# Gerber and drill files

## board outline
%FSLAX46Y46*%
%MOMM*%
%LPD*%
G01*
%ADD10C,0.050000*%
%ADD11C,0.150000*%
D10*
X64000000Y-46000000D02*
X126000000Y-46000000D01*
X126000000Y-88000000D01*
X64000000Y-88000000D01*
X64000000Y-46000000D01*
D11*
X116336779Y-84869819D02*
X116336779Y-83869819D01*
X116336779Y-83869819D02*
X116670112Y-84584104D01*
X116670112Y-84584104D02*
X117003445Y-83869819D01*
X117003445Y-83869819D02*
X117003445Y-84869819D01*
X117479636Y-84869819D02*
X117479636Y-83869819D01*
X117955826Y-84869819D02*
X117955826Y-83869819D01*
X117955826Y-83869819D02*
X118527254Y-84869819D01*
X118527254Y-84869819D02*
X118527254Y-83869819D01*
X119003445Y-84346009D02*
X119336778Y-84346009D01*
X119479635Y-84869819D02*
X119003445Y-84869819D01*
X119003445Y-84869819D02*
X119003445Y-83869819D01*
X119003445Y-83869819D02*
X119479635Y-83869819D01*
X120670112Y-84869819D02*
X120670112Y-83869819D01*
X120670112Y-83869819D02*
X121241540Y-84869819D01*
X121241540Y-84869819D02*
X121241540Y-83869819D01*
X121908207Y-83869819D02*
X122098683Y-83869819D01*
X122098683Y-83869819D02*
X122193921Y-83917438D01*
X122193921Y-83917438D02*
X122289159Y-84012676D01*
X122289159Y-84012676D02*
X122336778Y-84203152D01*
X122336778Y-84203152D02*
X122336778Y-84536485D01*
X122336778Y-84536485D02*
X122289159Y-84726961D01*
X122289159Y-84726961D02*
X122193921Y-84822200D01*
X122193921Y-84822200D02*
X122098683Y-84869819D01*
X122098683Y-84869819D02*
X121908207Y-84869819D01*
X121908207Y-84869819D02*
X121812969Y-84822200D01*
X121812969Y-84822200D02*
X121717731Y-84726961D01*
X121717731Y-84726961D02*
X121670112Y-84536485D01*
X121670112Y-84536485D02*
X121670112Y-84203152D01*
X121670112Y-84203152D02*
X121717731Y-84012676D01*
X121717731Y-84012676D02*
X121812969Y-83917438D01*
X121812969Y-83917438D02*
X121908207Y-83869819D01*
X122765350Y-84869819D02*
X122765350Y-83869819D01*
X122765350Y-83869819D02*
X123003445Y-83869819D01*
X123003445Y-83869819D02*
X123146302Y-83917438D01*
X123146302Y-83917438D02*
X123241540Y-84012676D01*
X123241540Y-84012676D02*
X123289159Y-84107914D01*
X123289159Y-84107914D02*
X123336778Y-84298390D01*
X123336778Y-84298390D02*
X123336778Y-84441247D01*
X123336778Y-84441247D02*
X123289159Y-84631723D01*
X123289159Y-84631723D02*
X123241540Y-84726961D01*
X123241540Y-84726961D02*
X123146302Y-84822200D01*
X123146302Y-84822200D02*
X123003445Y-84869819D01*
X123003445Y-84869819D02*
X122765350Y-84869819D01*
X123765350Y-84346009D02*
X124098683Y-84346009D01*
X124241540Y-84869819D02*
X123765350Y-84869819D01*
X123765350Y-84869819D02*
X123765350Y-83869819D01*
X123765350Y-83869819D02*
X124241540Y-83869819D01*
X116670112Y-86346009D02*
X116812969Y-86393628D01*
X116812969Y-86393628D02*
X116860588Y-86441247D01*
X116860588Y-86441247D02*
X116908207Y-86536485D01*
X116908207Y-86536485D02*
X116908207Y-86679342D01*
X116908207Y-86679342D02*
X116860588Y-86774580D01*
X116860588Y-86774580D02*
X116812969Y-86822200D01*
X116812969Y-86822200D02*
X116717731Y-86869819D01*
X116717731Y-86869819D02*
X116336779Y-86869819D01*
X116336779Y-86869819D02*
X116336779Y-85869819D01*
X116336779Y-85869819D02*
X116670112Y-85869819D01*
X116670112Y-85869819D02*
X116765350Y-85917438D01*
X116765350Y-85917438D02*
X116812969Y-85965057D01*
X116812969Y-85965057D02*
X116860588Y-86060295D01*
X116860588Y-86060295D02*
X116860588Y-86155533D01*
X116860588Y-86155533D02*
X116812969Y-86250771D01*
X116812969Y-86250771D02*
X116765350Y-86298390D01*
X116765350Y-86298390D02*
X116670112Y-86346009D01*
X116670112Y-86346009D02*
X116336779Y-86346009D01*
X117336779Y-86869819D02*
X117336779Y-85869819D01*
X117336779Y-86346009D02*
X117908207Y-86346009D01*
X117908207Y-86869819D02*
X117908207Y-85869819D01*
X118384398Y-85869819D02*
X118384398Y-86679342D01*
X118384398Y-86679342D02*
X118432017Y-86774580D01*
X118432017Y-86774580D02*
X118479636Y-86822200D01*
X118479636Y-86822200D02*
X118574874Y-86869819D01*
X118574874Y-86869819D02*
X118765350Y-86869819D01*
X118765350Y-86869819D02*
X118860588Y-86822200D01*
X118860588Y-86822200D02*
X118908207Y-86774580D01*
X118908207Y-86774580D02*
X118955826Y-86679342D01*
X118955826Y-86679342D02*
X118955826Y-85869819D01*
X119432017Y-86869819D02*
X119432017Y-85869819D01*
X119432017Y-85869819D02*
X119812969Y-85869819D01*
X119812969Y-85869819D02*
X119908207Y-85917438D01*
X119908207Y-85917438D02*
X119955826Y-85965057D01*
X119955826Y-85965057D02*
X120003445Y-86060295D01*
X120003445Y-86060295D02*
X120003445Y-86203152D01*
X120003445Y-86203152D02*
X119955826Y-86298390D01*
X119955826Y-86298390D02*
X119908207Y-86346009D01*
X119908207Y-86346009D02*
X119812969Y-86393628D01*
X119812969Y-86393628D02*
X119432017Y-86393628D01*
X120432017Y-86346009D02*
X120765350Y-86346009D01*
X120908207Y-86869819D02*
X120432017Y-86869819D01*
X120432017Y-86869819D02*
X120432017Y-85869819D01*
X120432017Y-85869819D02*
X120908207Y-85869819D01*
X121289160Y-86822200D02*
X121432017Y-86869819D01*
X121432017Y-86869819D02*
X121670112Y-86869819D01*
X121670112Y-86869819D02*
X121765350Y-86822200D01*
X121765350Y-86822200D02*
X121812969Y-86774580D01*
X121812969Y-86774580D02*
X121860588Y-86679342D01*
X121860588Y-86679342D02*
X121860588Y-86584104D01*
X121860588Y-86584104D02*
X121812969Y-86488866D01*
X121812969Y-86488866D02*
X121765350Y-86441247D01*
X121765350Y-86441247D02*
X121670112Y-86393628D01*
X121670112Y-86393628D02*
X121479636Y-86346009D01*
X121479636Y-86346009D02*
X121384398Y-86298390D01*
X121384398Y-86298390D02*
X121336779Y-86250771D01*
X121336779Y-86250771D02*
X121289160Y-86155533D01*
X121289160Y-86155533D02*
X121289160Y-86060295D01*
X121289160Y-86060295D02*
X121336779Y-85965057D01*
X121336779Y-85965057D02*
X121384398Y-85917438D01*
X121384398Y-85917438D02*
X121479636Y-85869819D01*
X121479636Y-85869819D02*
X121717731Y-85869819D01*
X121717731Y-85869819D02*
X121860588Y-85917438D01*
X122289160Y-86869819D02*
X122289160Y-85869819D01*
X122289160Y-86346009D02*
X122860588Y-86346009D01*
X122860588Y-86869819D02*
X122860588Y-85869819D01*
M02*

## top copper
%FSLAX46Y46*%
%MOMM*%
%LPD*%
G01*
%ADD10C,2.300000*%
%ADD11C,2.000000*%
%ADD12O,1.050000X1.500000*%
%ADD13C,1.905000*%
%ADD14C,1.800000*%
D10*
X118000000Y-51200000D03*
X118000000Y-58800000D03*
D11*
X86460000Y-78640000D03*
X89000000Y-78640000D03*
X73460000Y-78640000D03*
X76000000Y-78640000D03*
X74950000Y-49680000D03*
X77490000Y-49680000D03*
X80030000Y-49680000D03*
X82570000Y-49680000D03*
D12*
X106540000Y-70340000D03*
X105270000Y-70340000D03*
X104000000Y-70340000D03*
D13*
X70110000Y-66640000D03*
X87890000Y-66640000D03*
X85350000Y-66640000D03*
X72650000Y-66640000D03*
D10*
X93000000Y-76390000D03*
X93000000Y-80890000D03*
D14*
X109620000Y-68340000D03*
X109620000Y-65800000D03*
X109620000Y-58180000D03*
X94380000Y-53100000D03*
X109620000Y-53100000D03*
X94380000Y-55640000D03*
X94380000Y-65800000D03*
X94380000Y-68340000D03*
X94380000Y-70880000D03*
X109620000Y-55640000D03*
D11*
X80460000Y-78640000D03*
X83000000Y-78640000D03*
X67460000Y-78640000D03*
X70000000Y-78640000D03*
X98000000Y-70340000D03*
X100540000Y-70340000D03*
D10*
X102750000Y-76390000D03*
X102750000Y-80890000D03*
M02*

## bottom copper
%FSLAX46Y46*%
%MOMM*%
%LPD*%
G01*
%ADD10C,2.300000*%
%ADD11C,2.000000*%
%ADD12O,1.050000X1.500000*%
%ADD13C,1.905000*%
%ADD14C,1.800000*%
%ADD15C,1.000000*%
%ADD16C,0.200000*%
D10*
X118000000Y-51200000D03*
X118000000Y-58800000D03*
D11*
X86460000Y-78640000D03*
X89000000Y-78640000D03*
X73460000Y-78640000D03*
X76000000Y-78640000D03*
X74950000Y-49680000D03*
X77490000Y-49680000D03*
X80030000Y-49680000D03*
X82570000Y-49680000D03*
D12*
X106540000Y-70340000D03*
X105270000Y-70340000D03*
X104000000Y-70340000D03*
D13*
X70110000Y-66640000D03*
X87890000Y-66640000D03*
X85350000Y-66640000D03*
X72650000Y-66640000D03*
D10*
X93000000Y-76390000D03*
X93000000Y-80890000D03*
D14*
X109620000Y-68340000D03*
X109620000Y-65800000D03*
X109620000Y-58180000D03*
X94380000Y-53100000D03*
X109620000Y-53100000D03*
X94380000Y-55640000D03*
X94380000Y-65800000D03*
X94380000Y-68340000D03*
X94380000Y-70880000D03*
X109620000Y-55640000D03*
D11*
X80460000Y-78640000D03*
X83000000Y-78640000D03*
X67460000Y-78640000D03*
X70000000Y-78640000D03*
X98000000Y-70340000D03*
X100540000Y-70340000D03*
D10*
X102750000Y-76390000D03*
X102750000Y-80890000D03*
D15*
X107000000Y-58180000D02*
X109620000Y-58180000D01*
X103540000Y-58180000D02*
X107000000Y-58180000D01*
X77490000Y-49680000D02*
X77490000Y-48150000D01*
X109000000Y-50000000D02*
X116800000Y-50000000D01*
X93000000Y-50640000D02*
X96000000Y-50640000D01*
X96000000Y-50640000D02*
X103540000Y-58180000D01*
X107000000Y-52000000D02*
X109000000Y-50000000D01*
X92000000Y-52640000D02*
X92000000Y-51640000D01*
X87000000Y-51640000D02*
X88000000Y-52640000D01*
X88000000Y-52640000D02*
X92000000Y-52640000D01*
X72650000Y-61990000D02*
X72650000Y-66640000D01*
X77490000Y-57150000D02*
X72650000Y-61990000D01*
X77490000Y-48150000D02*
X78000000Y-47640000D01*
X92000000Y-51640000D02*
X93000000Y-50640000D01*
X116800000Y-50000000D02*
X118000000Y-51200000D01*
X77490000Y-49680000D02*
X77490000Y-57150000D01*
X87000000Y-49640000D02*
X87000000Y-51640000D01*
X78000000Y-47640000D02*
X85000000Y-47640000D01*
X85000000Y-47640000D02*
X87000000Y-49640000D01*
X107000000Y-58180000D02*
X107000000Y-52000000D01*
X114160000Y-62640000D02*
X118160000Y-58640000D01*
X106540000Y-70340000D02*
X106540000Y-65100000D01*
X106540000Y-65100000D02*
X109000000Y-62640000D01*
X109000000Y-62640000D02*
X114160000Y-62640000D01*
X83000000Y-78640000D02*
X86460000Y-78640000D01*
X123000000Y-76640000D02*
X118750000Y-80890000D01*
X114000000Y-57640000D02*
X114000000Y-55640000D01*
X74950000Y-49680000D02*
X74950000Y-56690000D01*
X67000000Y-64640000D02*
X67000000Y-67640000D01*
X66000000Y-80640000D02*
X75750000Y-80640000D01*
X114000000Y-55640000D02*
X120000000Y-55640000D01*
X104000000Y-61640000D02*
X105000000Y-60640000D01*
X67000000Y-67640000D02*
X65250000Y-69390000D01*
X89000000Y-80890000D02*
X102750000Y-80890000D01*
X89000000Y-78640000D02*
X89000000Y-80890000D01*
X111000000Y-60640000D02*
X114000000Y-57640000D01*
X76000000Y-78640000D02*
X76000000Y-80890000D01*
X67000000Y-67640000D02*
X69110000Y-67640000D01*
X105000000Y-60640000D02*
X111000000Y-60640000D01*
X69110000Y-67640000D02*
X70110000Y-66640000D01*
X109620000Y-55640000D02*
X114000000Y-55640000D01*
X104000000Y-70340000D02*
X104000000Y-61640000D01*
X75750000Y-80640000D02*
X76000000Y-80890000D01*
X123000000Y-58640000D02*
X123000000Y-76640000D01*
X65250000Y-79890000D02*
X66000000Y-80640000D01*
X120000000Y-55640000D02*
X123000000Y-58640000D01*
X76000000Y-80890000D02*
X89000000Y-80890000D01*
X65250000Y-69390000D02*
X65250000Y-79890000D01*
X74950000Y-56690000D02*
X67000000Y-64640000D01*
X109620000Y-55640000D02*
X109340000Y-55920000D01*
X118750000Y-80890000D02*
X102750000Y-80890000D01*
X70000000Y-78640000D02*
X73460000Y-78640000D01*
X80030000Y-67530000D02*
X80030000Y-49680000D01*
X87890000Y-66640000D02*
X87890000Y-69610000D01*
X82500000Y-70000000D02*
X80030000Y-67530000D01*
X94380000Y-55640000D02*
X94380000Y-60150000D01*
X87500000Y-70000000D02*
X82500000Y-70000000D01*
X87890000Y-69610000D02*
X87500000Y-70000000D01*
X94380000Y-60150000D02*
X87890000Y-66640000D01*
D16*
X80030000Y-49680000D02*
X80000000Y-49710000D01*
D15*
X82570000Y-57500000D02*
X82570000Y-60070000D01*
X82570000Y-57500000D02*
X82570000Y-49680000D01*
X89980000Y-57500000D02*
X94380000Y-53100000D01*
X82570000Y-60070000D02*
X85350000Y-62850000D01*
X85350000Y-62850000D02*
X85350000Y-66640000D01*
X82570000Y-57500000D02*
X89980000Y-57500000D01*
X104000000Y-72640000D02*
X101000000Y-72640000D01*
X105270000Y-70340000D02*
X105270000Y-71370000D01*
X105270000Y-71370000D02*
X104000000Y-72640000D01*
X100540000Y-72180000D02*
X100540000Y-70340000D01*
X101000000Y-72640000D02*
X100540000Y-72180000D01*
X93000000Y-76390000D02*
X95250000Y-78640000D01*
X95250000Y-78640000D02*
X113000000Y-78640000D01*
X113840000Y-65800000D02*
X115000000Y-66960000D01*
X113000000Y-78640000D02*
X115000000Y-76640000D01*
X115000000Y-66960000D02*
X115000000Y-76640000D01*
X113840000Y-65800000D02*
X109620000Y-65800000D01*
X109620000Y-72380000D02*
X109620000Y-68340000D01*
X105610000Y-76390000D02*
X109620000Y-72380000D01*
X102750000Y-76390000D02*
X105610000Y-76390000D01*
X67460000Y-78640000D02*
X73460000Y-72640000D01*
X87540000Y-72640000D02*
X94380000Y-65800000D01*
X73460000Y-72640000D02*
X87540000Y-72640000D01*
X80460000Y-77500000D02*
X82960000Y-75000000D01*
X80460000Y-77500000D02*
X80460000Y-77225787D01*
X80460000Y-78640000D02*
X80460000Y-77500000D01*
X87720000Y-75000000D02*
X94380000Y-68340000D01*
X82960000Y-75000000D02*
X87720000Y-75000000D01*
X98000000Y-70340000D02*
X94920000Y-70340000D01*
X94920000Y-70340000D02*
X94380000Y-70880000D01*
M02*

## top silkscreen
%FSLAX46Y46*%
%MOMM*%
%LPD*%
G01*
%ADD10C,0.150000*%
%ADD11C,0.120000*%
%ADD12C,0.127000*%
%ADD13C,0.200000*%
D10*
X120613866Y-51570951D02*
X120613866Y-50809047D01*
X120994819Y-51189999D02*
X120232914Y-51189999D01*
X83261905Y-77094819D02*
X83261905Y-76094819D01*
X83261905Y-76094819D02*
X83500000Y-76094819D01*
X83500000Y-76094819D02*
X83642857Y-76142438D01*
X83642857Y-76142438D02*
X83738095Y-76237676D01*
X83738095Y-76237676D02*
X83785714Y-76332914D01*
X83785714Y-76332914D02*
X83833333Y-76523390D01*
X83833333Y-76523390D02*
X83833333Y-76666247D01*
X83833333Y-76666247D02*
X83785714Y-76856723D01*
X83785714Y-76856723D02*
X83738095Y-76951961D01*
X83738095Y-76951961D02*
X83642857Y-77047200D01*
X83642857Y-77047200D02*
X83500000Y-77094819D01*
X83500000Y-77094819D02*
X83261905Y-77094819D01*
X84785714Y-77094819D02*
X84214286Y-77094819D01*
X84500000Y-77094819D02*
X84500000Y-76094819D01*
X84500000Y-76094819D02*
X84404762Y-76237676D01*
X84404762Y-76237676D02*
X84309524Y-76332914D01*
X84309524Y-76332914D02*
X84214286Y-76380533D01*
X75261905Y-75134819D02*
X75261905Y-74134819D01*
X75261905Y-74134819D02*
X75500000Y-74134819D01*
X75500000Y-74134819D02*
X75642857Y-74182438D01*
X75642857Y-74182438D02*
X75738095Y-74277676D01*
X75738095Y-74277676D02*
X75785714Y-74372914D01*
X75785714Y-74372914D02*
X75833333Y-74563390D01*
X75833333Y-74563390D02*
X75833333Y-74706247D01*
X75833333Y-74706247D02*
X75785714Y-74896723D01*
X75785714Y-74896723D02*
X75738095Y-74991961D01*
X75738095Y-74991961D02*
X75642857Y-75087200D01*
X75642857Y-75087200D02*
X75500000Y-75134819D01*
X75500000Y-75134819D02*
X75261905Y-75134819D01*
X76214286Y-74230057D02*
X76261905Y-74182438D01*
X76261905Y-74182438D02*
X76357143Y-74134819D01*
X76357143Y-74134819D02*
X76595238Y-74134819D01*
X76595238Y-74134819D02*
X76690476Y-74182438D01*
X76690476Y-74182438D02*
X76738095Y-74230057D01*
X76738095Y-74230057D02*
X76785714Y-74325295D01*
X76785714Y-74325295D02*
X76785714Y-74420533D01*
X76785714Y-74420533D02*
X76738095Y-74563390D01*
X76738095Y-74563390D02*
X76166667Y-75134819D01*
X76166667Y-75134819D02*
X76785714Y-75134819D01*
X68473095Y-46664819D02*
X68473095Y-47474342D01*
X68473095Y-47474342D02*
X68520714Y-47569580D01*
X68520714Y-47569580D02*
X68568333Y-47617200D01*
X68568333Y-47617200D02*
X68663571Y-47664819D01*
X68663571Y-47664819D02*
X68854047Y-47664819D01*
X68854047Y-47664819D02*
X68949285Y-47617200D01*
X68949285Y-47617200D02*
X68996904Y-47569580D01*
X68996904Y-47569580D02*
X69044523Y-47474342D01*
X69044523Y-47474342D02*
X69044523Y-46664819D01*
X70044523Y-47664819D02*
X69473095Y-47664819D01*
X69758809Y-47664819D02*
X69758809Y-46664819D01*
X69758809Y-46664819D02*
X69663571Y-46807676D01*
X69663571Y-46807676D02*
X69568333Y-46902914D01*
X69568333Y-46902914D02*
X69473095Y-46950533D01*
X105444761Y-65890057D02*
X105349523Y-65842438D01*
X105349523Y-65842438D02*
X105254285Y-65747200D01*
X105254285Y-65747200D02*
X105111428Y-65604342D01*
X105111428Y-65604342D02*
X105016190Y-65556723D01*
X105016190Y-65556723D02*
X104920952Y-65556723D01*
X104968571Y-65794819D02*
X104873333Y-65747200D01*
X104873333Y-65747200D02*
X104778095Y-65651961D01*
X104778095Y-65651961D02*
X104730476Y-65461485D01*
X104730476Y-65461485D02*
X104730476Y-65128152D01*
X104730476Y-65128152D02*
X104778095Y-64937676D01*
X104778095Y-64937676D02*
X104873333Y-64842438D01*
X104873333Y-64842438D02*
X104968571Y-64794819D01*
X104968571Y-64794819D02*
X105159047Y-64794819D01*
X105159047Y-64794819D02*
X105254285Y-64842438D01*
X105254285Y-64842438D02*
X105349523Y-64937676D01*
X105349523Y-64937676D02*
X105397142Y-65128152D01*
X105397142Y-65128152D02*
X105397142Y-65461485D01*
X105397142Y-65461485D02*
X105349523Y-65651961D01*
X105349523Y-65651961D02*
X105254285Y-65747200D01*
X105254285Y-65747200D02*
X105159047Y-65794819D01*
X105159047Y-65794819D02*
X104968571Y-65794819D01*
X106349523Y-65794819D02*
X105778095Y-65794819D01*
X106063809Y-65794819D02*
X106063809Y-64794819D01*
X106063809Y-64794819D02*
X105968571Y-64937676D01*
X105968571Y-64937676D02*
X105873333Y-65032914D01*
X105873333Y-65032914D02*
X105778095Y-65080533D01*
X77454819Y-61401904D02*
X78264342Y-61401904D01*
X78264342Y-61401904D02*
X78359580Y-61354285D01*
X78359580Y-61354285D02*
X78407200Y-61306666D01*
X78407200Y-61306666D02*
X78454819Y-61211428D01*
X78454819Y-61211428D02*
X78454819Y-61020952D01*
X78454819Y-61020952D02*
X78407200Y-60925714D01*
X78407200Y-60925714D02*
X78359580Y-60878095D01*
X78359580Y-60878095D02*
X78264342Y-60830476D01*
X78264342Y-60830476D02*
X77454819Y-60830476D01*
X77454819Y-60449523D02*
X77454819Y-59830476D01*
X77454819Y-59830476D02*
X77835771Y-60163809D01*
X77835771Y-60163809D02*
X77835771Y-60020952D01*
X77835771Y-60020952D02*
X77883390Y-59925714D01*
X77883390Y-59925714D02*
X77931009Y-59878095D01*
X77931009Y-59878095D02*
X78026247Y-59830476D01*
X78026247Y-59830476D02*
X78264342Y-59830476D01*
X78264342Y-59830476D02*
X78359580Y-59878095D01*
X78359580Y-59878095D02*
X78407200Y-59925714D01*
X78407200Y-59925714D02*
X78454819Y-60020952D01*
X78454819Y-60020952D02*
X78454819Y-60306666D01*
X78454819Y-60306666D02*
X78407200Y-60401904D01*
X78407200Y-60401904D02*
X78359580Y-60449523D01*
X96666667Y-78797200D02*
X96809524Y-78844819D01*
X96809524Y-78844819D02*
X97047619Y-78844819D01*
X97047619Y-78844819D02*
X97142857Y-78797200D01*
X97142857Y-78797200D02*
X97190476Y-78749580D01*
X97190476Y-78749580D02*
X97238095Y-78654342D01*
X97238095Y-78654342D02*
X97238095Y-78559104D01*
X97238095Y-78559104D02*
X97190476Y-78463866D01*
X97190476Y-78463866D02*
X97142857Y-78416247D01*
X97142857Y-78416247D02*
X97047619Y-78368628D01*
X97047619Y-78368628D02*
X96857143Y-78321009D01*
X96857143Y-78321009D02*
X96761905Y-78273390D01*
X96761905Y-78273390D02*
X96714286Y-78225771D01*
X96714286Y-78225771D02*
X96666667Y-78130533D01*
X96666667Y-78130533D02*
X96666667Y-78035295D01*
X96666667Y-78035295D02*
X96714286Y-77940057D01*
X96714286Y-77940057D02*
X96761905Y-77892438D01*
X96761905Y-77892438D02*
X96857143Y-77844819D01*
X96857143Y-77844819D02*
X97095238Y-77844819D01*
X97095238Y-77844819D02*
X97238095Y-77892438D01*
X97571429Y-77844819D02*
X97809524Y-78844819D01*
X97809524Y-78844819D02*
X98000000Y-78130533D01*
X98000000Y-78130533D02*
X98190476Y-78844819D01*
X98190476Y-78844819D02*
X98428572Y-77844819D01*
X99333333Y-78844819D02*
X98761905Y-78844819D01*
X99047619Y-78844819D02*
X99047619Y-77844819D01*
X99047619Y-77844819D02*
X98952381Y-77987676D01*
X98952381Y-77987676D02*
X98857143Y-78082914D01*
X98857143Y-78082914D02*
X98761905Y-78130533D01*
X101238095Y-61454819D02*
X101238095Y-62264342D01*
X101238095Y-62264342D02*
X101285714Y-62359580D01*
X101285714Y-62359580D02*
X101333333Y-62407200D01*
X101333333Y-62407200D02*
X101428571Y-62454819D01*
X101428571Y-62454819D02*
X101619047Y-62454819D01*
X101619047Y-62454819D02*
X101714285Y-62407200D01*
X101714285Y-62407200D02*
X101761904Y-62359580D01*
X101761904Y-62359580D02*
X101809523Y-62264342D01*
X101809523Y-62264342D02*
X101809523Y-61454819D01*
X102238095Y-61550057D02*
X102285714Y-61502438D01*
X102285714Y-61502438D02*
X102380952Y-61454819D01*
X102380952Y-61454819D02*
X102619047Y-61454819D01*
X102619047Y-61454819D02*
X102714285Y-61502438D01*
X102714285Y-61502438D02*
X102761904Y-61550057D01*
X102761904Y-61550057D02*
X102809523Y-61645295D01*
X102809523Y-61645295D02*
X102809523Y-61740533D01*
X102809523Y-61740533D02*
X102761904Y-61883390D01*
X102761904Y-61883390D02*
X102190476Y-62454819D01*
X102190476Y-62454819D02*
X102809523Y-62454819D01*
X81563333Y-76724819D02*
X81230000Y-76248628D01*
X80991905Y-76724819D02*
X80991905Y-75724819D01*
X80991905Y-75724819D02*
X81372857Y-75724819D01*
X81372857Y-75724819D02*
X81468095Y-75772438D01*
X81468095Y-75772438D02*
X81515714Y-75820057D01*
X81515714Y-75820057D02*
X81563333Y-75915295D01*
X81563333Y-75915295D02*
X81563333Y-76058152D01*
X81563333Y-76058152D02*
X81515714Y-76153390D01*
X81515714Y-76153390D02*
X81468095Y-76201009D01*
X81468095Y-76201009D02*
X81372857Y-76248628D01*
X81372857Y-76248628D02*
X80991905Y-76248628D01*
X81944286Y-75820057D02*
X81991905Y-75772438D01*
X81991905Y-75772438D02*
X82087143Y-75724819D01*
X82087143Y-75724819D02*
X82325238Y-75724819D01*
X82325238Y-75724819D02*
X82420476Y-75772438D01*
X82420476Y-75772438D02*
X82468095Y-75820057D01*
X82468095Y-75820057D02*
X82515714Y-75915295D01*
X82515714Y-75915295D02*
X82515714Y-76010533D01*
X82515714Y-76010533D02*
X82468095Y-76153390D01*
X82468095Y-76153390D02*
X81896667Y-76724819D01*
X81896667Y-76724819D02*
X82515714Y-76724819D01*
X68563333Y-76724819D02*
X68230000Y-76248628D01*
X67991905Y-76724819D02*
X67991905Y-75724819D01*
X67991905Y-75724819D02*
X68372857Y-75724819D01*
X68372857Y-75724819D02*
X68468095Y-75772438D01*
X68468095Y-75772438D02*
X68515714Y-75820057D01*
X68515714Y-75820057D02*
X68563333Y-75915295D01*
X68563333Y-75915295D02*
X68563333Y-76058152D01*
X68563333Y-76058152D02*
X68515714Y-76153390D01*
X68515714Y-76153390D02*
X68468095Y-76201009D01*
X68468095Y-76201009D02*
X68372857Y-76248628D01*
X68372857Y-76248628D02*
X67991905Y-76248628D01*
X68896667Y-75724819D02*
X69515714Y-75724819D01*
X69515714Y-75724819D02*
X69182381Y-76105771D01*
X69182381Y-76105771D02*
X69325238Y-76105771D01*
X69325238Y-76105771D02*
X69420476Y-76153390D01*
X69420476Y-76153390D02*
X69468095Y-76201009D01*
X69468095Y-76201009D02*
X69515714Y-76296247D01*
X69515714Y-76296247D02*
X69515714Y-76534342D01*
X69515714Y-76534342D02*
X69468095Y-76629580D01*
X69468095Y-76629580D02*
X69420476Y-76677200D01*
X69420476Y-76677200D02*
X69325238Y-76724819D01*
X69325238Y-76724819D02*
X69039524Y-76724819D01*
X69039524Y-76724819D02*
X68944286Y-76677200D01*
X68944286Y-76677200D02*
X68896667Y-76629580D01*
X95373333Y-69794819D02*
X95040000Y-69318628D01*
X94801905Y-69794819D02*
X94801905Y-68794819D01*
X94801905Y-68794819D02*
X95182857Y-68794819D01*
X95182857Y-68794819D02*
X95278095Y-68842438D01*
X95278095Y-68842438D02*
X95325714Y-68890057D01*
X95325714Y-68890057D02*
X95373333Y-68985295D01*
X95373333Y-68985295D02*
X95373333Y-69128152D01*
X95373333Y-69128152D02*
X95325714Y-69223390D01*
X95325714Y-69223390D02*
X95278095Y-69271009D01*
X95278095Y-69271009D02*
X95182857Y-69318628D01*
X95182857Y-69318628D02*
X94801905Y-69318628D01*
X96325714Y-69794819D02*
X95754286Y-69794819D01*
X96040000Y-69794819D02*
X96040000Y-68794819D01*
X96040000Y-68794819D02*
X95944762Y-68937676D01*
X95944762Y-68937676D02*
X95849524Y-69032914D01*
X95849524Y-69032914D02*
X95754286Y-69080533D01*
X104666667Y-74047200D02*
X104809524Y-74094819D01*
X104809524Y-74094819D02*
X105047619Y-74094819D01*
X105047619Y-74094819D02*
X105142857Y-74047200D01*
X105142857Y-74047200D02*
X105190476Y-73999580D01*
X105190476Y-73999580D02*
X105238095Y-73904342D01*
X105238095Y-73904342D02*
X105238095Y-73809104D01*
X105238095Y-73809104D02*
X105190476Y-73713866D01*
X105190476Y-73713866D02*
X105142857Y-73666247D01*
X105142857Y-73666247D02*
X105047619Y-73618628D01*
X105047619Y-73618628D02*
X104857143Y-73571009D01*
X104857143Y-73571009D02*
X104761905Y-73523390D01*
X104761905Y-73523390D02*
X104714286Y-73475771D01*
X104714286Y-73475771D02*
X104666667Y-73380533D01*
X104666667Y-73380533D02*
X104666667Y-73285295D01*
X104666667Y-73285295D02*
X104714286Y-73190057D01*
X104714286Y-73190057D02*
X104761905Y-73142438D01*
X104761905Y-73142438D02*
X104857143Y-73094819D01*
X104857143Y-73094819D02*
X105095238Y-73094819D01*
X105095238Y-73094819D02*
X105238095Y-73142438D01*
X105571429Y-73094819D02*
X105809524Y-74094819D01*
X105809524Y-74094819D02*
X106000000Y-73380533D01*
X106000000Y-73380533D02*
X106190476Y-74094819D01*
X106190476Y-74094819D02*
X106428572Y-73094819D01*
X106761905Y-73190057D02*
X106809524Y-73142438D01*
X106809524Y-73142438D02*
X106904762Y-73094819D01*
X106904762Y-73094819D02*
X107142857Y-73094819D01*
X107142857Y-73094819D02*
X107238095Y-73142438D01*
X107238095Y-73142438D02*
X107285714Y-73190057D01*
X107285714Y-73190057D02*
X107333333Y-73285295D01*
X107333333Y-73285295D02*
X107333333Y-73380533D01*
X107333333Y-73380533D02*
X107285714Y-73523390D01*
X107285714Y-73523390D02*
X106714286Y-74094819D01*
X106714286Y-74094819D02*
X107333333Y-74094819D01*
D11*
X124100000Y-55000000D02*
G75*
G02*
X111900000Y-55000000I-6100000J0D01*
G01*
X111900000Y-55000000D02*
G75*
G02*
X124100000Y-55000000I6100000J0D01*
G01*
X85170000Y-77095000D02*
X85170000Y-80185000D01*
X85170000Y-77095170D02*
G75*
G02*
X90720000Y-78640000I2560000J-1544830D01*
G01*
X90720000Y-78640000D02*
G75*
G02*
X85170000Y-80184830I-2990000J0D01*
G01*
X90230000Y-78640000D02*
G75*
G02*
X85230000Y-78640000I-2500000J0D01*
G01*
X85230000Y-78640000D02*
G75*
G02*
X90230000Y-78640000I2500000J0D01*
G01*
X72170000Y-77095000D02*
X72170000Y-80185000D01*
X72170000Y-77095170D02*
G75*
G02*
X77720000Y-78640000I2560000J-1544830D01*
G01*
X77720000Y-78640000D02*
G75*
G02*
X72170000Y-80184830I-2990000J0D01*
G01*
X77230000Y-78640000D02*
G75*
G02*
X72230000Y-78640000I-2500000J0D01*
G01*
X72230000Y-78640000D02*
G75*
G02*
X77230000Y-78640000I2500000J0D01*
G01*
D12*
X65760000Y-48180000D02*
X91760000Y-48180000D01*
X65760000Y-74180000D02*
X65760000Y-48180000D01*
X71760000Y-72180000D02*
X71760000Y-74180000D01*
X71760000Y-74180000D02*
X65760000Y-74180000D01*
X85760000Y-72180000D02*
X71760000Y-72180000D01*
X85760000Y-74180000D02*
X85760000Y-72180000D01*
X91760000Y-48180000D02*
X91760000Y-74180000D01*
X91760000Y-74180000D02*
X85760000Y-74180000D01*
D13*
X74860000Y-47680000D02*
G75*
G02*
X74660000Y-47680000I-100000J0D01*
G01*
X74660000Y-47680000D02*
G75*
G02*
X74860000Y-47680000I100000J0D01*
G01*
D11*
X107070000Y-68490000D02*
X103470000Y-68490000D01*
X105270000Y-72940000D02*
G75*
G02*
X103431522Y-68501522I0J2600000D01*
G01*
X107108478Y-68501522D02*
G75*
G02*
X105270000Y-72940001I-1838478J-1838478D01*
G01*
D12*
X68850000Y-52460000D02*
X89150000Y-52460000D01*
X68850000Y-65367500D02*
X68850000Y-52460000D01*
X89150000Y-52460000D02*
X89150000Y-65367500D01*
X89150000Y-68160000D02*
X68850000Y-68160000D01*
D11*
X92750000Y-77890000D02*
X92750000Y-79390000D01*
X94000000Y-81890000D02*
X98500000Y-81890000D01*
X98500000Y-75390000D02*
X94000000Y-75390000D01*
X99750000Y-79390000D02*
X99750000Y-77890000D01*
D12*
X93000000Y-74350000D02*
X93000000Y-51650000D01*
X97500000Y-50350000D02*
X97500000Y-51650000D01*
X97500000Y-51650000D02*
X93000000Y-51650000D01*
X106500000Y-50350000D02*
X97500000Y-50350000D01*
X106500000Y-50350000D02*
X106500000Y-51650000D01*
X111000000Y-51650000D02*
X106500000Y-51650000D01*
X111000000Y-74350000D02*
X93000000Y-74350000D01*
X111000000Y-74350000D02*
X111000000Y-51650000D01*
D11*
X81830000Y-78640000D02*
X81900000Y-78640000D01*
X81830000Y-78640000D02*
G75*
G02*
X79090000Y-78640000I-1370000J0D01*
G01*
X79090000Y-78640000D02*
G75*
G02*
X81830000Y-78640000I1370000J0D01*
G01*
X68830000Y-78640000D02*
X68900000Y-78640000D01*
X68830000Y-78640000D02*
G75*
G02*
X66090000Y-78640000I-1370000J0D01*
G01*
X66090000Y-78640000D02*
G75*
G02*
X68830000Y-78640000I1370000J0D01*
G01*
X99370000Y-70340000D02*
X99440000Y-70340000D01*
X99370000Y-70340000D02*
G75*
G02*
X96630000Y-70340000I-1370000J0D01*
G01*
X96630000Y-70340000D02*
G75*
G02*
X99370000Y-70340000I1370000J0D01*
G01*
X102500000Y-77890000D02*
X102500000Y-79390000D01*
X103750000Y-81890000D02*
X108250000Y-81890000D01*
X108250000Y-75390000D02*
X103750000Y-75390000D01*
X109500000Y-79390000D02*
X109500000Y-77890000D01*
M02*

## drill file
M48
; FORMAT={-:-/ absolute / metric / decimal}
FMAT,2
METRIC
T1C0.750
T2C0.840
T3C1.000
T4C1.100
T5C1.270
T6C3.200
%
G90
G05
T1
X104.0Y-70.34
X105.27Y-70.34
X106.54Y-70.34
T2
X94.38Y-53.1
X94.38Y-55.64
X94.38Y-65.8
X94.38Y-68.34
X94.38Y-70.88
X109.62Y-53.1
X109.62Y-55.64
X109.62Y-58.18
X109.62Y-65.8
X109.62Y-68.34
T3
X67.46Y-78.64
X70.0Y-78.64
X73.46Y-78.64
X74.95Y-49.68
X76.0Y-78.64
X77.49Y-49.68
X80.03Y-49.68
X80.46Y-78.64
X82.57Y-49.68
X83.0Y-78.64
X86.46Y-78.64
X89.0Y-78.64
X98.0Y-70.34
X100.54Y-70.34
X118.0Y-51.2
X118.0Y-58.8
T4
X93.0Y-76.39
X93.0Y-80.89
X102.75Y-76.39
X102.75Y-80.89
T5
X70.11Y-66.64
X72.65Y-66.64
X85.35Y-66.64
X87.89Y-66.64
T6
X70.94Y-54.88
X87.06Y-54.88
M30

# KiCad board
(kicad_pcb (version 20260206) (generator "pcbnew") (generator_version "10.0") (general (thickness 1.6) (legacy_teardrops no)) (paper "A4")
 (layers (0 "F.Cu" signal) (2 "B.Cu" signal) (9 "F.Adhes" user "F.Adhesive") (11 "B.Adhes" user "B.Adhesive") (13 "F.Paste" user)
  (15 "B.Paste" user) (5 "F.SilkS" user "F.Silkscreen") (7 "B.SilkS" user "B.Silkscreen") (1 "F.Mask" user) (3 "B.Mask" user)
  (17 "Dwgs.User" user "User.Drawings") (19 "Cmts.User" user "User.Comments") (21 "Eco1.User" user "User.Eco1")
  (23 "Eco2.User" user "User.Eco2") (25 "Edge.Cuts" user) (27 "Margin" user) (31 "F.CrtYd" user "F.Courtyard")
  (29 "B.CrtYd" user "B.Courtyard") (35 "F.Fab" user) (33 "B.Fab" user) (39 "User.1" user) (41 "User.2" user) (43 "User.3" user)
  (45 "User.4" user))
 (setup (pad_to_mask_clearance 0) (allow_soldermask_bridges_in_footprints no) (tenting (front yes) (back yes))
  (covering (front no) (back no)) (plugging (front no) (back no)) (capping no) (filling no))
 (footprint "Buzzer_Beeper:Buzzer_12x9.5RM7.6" (layer "F.Cu") (at 118 51.2 -90)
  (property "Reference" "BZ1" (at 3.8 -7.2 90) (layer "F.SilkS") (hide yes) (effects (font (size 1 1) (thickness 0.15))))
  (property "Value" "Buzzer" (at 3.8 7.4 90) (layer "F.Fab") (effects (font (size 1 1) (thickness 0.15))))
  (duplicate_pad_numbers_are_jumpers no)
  (fp_circle (center 3.8 0) (end 9.9 0) (stroke (width 0.12) (type solid)) (fill no) (layer "F.SilkS"))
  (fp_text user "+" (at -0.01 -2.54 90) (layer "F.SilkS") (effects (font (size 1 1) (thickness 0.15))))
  (pad "1" thru_hole circle (at 0 0 270) (size 2.3 2.3) (drill 1) (layers "*.Cu" "*.Mask") (remove_unused_layers no) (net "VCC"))
  (pad "2" thru_hole circle (at 7.6 0 270) (size 2.3 2.3) (drill 1) (layers "*.Cu" "*.Mask") (remove_unused_layers no) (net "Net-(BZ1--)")))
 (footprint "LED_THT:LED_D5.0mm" (layer "F.Cu") (at 86.46 78.64)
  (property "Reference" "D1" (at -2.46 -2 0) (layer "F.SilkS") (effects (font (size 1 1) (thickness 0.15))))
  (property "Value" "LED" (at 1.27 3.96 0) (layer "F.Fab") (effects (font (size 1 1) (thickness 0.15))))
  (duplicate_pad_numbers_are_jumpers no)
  (fp_line (start -1.29 -1.545) (end -1.29 1.545) (stroke (width 0.12) (type solid)) (layer "F.SilkS"))
  (fp_arc (start -1.29 -1.54483) (mid 2.071779 -2.880495) (end 4.26 0) (stroke (width 0.12) (type solid)) (layer "F.SilkS"))
  (fp_arc (start 4.26 0) (mid 2.071779 2.880495) (end -1.29 1.54483) (stroke (width 0.12) (type solid)) (layer "F.SilkS"))
  (fp_circle (center 1.27 0) (end 3.77 0) (stroke (width 0.12) (type solid)) (fill no) (layer "F.SilkS"))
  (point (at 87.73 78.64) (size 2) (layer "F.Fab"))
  (pad "1" thru_hole circle (at 0 0) (size 2 2) (drill 1) (layers "*.Cu" "*.Mask") (remove_unused_layers no) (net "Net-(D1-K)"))
  (pad "2" thru_hole circle (at 2.54 0) (size 2 2) (drill 1) (layers "*.Cu" "*.Mask") (remove_unused_layers no) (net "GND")))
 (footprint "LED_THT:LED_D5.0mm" (layer "F.Cu") (at 73.46 78.64)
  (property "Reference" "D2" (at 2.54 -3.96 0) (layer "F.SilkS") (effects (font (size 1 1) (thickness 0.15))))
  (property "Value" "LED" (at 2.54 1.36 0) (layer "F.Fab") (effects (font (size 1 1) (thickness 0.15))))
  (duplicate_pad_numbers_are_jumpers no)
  (fp_line (start -1.29 -1.545) (end -1.29 1.545) (stroke (width 0.12) (type solid)) (layer "F.SilkS"))
  (fp_arc (start -1.29 -1.54483) (mid 2.071779 -2.880495) (end 4.26 0) (stroke (width 0.12) (type solid)) (layer "F.SilkS"))
  (fp_arc (start 4.26 0) (mid 2.071779 2.880495) (end -1.29 1.54483) (stroke (width 0.12) (type solid)) (layer "F.SilkS"))
  (fp_circle (center 1.27 0) (end 3.77 0) (stroke (width 0.12) (type solid)) (fill no) (layer "F.SilkS"))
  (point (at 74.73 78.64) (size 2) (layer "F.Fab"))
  (pad "1" thru_hole circle (at 0 0) (size 2 2) (drill 1) (layers "*.Cu" "*.Mask") (remove_unused_layers no) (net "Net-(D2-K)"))
  (pad "2" thru_hole circle (at 2.54 0) (size 2 2) (drill 1) (layers "*.Cu" "*.Mask") (remove_unused_layers no) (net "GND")))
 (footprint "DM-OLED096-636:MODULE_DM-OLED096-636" (layer "F.Cu") (at 78.76 61.18)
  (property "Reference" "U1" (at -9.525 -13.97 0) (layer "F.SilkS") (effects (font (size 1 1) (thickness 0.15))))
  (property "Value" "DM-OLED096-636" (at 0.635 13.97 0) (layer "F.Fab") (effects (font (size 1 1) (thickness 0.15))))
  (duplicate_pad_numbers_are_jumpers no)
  (fp_line (start -13 -13) (end 13 -13) (stroke (width 0.127) (type solid)) (layer "F.SilkS"))
  (fp_line (start -13 13) (end -13 -13) (stroke (width 0.127) (type solid)) (layer "F.SilkS"))
  (fp_line (start -7 11) (end -7 13) (stroke (width 0.127) (type solid)) (layer "F.SilkS"))
  (fp_line (start -7 13) (end -13 13) (stroke (width 0.127) (type solid)) (layer "F.SilkS"))
  (fp_line (start 7 11) (end -7 11) (stroke (width 0.127) (type solid)) (layer "F.SilkS"))
  (fp_line (start 7 13) (end 7 11) (stroke (width 0.127) (type solid)) (layer "F.SilkS"))
  (fp_line (start 13 -13) (end 13 13) (stroke (width 0.127) (type solid)) (layer "F.SilkS"))
  (fp_line (start 13 13) (end 7 13) (stroke (width 0.127) (type solid)) (layer "F.SilkS"))
  (fp_circle (center -4 -13.5) (end -3.9 -13.5) (stroke (width 0.2) (type solid)) (fill no) (layer "F.SilkS"))
  (pad "1" thru_hole circle (at -3.81 -11.5) (size 2 2) (drill 1) (layers "*.Cu" "*.Mask") (remove_unused_layers no) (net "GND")
   (solder_mask_margin 0.102))
  (pad "2" thru_hole circle (at -1.27 -11.5) (size 2 2) (drill 1) (layers "*.Cu" "*.Mask") (remove_unused_layers no) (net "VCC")
   (solder_mask_margin 0.102))
  (pad "3" thru_hole circle (at 1.27 -11.5) (size 2 2) (drill 1) (layers "*.Cu" "*.Mask") (remove_unused_layers no) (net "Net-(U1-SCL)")
   (solder_mask_margin 0.102))
  (pad "4" thru_hole circle (at 3.81 -11.5) (size 2 2) (drill 1) (layers "*.Cu" "*.Mask") (remove_unused_layers no) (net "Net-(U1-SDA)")
   (solder_mask_margin 0.102)))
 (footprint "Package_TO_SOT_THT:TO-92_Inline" (layer "F.Cu") (at 106.54 70.34 180)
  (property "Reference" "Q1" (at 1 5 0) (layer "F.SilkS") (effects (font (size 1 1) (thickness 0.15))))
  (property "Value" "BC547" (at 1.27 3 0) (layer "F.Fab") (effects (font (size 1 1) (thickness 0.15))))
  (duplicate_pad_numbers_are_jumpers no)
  (fp_line (start -0.53 1.85) (end 3.07 1.85) (stroke (width 0.12) (type solid)) (layer "F.SilkS"))
  (fp_arc (start 1.27 -2.6) (mid 3.672087 -0.994977) (end 3.108478 1.838478) (stroke (width 0.12) (type solid)) (layer "F.SilkS"))
  (fp_arc (start -0.568478 1.838478) (mid -1.132087 -0.994977) (end 1.27 -2.6) (stroke (width 0.12) (type solid)) (layer "F.SilkS"))
  (pad "1" thru_hole oval (at 0 0 180) (size 1.05 1.5) (drill 0.75) (layers "*.Cu" "*.Mask") (remove_unused_layers no) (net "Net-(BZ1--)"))
  (pad "2" thru_hole oval (at 1.27 0 180) (size 1.05 1.5) (drill 0.75) (layers "*.Cu" "*.Mask") (remove_unused_layers no) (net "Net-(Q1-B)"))
  (pad "3" thru_hole oval (at 2.54 0 180) (size 1.05 1.5) (drill 0.75) (layers "*.Cu" "*.Mask") (remove_unused_layers no) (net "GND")))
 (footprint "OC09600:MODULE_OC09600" (layer "F.Cu") (at 79 60.31 90)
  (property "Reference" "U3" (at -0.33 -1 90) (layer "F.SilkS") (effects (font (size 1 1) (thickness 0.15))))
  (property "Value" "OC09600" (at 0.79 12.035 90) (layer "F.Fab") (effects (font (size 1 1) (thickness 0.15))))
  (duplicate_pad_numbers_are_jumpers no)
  (fp_line (start 7.85 -10.15) (end 7.85 10.15) (stroke (width 0.127) (type solid)) (layer "F.SilkS"))
  (fp_line (start -5.0575 -10.15) (end 7.85 -10.15) (stroke (width 0.127) (type solid)) (layer "F.SilkS"))
  (fp_line (start 7.85 10.15) (end -5.0575 10.15) (stroke (width 0.127) (type solid)) (layer "F.SilkS"))
  (fp_line (start -7.85 10.15) (end -7.85 -10.15) (stroke (width 0.127) (type solid)) (layer "F.SilkS"))
  (pad "" np_thru_hole circle (at 5.43 -8.06 90) (size 3.2 3.2) (drill 3.2) (layers "*.Cu" "*.Mask"))
  (pad "" np_thru_hole circle (at 5.43 8.06 90) (size 3.2 3.2) (drill 3.2) (layers "*.Cu" "*.Mask"))
  (pad "GND" thru_hole circle (at -6.33 -8.89 90) (size 1.905 1.905) (drill 1.27) (layers "*.Cu" "*.Mask") (remove_unused_layers no)
   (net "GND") (solder_mask_margin 0.102))
  (pad "SCL" thru_hole circle (at -6.33 8.89 90) (size 1.905 1.905) (drill 1.27) (layers "*.Cu" "*.Mask") (remove_unused_layers no)
   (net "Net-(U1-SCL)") (solder_mask_margin 0.102))
  (pad "SDA" thru_hole circle (at -6.33 6.35 90) (size 1.905 1.905) (drill 1.27) (layers "*.Cu" "*.Mask") (remove_unused_layers no)
   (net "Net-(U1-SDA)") (solder_mask_margin 0.102))
  (pad "VCC" thru_hole circle (at -6.33 -6.35 90) (size 1.905 1.905) (drill 1.27) (layers "*.Cu" "*.Mask") (remove_unused_layers no)
   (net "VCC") (solder_mask_margin 0.102)))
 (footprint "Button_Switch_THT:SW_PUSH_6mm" (layer "F.Cu") (at 93 76.39)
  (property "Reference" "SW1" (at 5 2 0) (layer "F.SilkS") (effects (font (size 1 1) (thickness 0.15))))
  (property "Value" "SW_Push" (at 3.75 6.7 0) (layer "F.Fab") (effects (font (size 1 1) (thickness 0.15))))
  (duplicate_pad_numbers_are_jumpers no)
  (fp_line (start -0.25 1.5) (end -0.25 3) (stroke (width 0.12) (type solid)) (layer "F.SilkS"))
  (fp_line (start 1 5.5) (end 5.5 5.5) (stroke (width 0.12) (type solid)) (layer "F.SilkS"))
  (fp_line (start 5.5 -1) (end 1 -1) (stroke (width 0.12) (type solid)) (layer "F.SilkS"))
  (fp_line (start 6.75 3) (end 6.75 1.5) (stroke (width 0.12) (type solid)) (layer "F.SilkS"))
  (pad "1" thru_hole circle (at 0 0 90) (size 2.3 2.3) (drill 1.1) (layers "*.Cu" "*.Mask") (remove_unused_layers no) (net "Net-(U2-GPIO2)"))
  (pad "2" thru_hole circle (at 0 4.5 90) (size 2.3 2.3) (drill 1.1) (layers "*.Cu" "*.Mask") (remove_unused_layers no) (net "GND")))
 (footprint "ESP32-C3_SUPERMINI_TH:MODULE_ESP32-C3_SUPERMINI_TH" (layer "F.Cu") (at 102 63)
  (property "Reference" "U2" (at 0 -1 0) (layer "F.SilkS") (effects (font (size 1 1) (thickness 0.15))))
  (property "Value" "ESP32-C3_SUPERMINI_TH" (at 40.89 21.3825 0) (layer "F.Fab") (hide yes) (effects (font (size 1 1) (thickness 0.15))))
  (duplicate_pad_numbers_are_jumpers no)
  (fp_line (start -9 11.35) (end -9 -11.35) (stroke (width 0.127) (type solid)) (layer "F.SilkS"))
  (fp_line (start -4.5 -12.65) (end -4.5 -11.35) (stroke (width 0.127) (type solid)) (layer "F.SilkS"))
  (fp_line (start -4.5 -11.35) (end -9 -11.35) (stroke (width 0.127) (type solid)) (layer "F.SilkS"))
  (fp_line (start 4.5 -12.65) (end -4.5 -12.65) (stroke (width 0.127) (type solid)) (layer "F.SilkS"))
  (fp_line (start 4.5 -12.65) (end 4.5 -11.35) (stroke (width 0.127) (type solid)) (layer "F.SilkS"))
  (fp_line (start 9 -11.35) (end 4.5 -11.35) (stroke (width 0.127) (type solid)) (layer "F.SilkS"))
  (fp_line (start 9 11.35) (end -9 11.35) (stroke (width 0.127) (type solid)) (layer "F.SilkS"))
  (fp_line (start 9 11.35) (end 9 -11.35) (stroke (width 0.127) (type solid)) (layer "F.SilkS"))
  (pad "1" thru_hole circle (at 7.62 5.34) (size 1.8 1.8) (drill 0.84) (layers "*.Cu" "*.Mask") (remove_unused_layers no)
   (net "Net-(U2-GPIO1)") (solder_mask_margin 0.102))
  (pad "2" thru_hole circle (at 7.62 2.8) (size 1.8 1.8) (drill 0.84) (layers "*.Cu" "*.Mask") (remove_unused_layers no)
   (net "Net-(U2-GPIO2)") (solder_mask_margin 0.102))
  (pad "3.3" thru_hole circle (at 7.62 -4.82) (size 1.8 1.8) (drill 0.84) (layers "*.Cu" "*.Mask") (remove_unused_layers no) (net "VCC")
   (solder_mask_margin 0.102))
  (pad "5" thru_hole circle (at -7.62 -9.9) (size 1.8 1.8) (drill 0.84) (layers "*.Cu" "*.Mask") (remove_unused_layers no)
   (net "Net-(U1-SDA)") (solder_mask_margin 0.102))
  (pad "5V" thru_hole circle (at 7.62 -9.9) (size 1.8 1.8) (drill 0.84) (layers "*.Cu" "*.Mask") (remove_unused_layers no)
   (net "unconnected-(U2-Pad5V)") (solder_mask_margin 0.102))
  (pad "6" thru_hole circle (at -7.62 -7.36) (size 1.8 1.8) (drill 0.84) (layers "*.Cu" "*.Mask") (remove_unused_layers no)
   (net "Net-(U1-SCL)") (solder_mask_margin 0.102))
  (pad "10" thru_hole circle (at -7.62 2.8) (size 1.8 1.8) (drill 0.84) (layers "*.Cu" "*.Mask") (remove_unused_layers no)
   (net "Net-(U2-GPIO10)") (solder_mask_margin 0.102))
  (pad "20" thru_hole circle (at -7.62 5.34) (size 1.8 1.8) (drill 0.84) (layers "*.Cu" "*.Mask") (remove_unused_layers no)
   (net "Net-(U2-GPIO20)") (solder_mask_margin 0.102))
  (pad "21" thru_hole circle (at -7.62 7.88) (size 1.8 1.8) (drill 0.84) (layers "*.Cu" "*.Mask") (remove_unused_layers no)
   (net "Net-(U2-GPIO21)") (solder_mask_margin 0.102))
  (pad "G" thru_hole circle (at 7.62 -7.36) (size 1.8 1.8) (drill 0.84) (layers "*.Cu" "*.Mask") (remove_unused_layers no) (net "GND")
   (solder_mask_margin 0.102)))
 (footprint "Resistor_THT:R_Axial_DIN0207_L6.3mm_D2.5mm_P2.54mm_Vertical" (layer "F.Cu") (at 80.46 78.64)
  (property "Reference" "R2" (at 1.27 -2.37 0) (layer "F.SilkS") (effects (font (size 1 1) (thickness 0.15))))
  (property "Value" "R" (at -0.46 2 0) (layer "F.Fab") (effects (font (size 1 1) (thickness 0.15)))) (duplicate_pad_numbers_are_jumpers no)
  (fp_line (start 1.37 0) (end 1.44 0) (stroke (width 0.12) (type solid)) (layer "F.SilkS"))
  (fp_circle (center 0 0) (end 1.37 0) (stroke (width 0.12) (type solid)) (fill no) (layer "F.SilkS"))
  (pad "1" thru_hole circle (at 0 0) (size 2 2) (drill 1) (layers "*.Cu" "*.Mask") (remove_unused_layers no) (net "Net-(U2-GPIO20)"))
  (pad "2" thru_hole circle (at 2.54 0) (size 2 2) (drill 1) (layers "*.Cu" "*.Mask") (remove_unused_layers no) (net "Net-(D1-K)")))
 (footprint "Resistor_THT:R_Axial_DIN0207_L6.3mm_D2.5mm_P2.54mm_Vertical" (layer "F.Cu") (at 67.46 78.64)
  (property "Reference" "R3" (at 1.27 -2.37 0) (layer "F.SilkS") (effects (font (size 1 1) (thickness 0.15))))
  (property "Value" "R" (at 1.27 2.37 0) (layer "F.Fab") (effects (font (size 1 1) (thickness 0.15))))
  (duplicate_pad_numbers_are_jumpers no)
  (fp_line (start 1.37 0) (end 1.44 0) (stroke (width 0.12) (type solid)) (layer "F.SilkS"))
  (fp_circle (center 0 0) (end 1.37 0) (stroke (width 0.12) (type solid)) (fill no) (layer "F.SilkS"))
  (pad "1" thru_hole circle (at 0 0) (size 2 2) (drill 1) (layers "*.Cu" "*.Mask") (remove_unused_layers no) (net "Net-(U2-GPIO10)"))
  (pad "2" thru_hole circle (at 2.54 0) (size 2 2) (drill 1) (layers "*.Cu" "*.Mask") (remove_unused_layers no) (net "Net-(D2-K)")))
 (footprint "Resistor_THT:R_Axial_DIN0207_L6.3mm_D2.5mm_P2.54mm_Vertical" (layer "F.Cu") (at 98 70.34)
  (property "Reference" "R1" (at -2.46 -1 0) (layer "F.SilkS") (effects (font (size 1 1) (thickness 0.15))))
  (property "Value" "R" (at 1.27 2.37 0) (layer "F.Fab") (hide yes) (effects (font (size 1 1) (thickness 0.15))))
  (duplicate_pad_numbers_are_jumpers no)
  (fp_line (start 1.37 0) (end 1.44 0) (stroke (width 0.12) (type solid)) (layer "F.SilkS"))
  (fp_circle (center 0 0) (end 1.37 0) (stroke (width 0.12) (type solid)) (fill no) (layer "F.SilkS"))
  (pad "1" thru_hole circle (at 0 0) (size 2 2) (drill 1) (layers "*.Cu" "*.Mask") (remove_unused_layers no) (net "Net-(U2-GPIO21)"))
  (pad "2" thru_hole circle (at 2.54 0) (size 2 2) (drill 1) (layers "*.Cu" "*.Mask") (remove_unused_layers no) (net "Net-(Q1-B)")))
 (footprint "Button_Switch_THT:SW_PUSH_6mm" (layer "F.Cu") (at 102.75 76.39)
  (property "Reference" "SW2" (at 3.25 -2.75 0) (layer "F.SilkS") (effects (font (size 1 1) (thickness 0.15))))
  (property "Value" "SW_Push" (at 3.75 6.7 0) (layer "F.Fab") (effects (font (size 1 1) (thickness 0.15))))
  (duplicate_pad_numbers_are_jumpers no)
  (fp_line (start -0.25 1.5) (end -0.25 3) (stroke (width 0.12) (type solid)) (layer "F.SilkS"))
  (fp_line (start 1 5.5) (end 5.5 5.5) (stroke (width 0.12) (type solid)) (layer "F.SilkS"))
  (fp_line (start 5.5 -1) (end 1 -1) (stroke (width 0.12) (type solid)) (layer "F.SilkS"))
  (fp_line (start 6.75 3) (end 6.75 1.5) (stroke (width 0.12) (type solid)) (layer "F.SilkS"))
  (pad "1" thru_hole circle (at 0 0 90) (size 2.3 2.3) (drill 1.1) (layers "*.Cu" "*.Mask") (remove_unused_layers no) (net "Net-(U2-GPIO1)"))
  (pad "2" thru_hole circle (at 0 4.5 90) (size 2.3 2.3) (drill 1.1) (layers "*.Cu" "*.Mask") (remove_unused_layers no) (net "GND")))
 (gr_rect (start 64 46) (end 126 88) (stroke (width 0.05) (type default)) (fill no) (layer "Edge.Cuts"))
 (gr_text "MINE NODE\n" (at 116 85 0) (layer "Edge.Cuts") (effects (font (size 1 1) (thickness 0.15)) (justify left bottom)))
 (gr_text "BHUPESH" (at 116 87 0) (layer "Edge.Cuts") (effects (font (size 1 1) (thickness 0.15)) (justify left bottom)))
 (segment (start 107 58.18) (end 109.62 58.18) (width 1) (layer "B.Cu") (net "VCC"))
 (segment (start 103.54 58.18) (end 107 58.18) (width 1) (layer "B.Cu") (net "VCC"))
 (segment (start 77.49 49.68) (end 77.49 48.15) (width 1) (layer "B.Cu") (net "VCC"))
 (segment (start 109 50) (end 116.8 50) (width 1) (layer "B.Cu") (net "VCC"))
 (segment (start 93 50.64) (end 96 50.64) (width 1) (layer "B.Cu") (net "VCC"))
 (segment (start 96 50.64) (end 103.54 58.18) (width 1) (layer "B.Cu") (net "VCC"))
 (segment (start 107 52) (end 109 50) (width 1) (layer "B.Cu") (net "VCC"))
 (segment (start 92 52.64) (end 92 51.64) (width 1) (layer "B.Cu") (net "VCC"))
 (segment (start 87 51.64) (end 88 52.64) (width 1) (layer "B.Cu") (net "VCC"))
 (segment (start 88 52.64) (end 92 52.64) (width 1) (layer "B.Cu") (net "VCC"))
 (segment (start 72.65 61.99) (end 72.65 66.64) (width 1) (layer "B.Cu") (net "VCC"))
 (segment (start 77.49 57.15) (end 72.65 61.99) (width 1) (layer "B.Cu") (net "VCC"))
 (segment (start 77.49 48.15) (end 78 47.64) (width 1) (layer "B.Cu") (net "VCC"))
 (segment (start 92 51.64) (end 93 50.64) (width 1) (layer "B.Cu") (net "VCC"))
 (segment (start 116.8 50) (end 118 51.2) (width 1) (layer "B.Cu") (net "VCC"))
 (segment (start 77.49 49.68) (end 77.49 57.15) (width 1) (layer "B.Cu") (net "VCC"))
 (segment (start 87 49.64) (end 87 51.64) (width 1) (layer "B.Cu") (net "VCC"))
 (segment (start 78 47.64) (end 85 47.64) (width 1) (layer "B.Cu") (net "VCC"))
 (segment (start 85 47.64) (end 87 49.64) (width 1) (layer "B.Cu") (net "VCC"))
 (segment (start 107 58.18) (end 107 52) (width 1) (layer "B.Cu") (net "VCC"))
 (segment (start 114.16 62.64) (end 118.16 58.64) (width 1) (layer "B.Cu") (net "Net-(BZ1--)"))
 (segment (start 106.54 70.34) (end 106.54 65.1) (width 1) (layer "B.Cu") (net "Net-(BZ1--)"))
 (segment (start 106.54 65.1) (end 109 62.64) (width 1) (layer "B.Cu") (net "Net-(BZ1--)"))
 (segment (start 109 62.64) (end 114.16 62.64) (width 1) (layer "B.Cu") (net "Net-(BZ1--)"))
 (segment (start 83 78.64) (end 86.46 78.64) (width 1) (layer "B.Cu") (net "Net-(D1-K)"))
 (segment (start 123 76.64) (end 118.75 80.89) (width 1) (layer "B.Cu") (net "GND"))
 (segment (start 114 57.64) (end 114 55.64) (width 1) (layer "B.Cu") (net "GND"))
 (segment (start 74.95 49.68) (end 74.95 56.69) (width 1) (layer "B.Cu") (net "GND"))
 (segment (start 67 64.64) (end 67 67.64) (width 1) (layer "B.Cu") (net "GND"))
 (segment (start 66 80.64) (end 75.75 80.64) (width 1) (layer "B.Cu") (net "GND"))
 (segment (start 114 55.64) (end 120 55.64) (width 1) (layer "B.Cu") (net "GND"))
 (segment (start 104 61.64) (end 105 60.64) (width 1) (layer "B.Cu") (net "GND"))
 (segment (start 67 67.64) (end 65.25 69.39) (width 1) (layer "B.Cu") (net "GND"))
 (segment (start 89 80.89) (end 102.75 80.89) (width 1) (layer "B.Cu") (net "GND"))
 (segment (start 89 78.64) (end 89 80.89) (width 1) (layer "B.Cu") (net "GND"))
 (segment (start 111 60.64) (end 114 57.64) (width 1) (layer "B.Cu") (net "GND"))
 (segment (start 76 78.64) (end 76 80.89) (width 1) (layer "B.Cu") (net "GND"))
 (segment (start 67 67.64) (end 69.11 67.64) (width 1) (layer "B.Cu") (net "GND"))
 (segment (start 105 60.64) (end 111 60.64) (width 1) (layer "B.Cu") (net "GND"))
 (segment (start 69.11 67.64) (end 70.11 66.64) (width 1) (layer "B.Cu") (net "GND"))
 (segment (start 109.62 55.64) (end 114 55.64) (width 1) (layer "B.Cu") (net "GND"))
 (segment (start 104 70.34) (end 104 61.64) (width 1) (layer "B.Cu") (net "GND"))
 (segment (start 75.75 80.64) (end 76 80.89) (width 1) (layer "B.Cu") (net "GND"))
 (segment (start 123 58.64) (end 123 76.64) (width 1) (layer "B.Cu") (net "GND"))
 (segment (start 65.25 79.89) (end 66 80.64) (width 1) (layer "B.Cu") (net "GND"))
 (segment (start 120 55.64) (end 123 58.64) (width 1) (layer "B.Cu") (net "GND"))
 (segment (start 76 80.89) (end 89 80.89) (width 1) (layer "B.Cu") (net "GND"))
 (segment (start 65.25 69.39) (end 65.25 79.89) (width 1) (layer "B.Cu") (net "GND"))
 (segment (start 74.95 56.69) (end 67 64.64) (width 1) (layer "B.Cu") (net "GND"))
 (segment (start 109.62 55.64) (end 109.34 55.92) (width 1) (layer "B.Cu") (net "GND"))
 (segment (start 118.75 80.89) (end 102.75 80.89) (width 1) (layer "B.Cu") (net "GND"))
 (segment (start 70 78.64) (end 73.46 78.64) (width 1) (layer "B.Cu") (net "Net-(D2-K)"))
 (segment (start 80.03 67.53) (end 80.03 49.68) (width 1) (layer "B.Cu") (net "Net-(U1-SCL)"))
 (segment (start 87.89 66.64) (end 87.89 69.61) (width 1) (layer "B.Cu") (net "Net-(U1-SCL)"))
 (segment (start 82.5 70) (end 80.03 67.53) (width 1) (layer "B.Cu") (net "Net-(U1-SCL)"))
 (segment (start 94.38 55.64) (end 94.38 60.15) (width 1) (layer "B.Cu") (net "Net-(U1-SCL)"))
 (segment (start 87.5 70) (end 82.5 70) (width 1) (layer "B.Cu") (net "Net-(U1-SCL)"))
 (segment (start 87.89 69.61) (end 87.5 70) (width 1) (layer "B.Cu") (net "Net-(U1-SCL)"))
 (segment (start 94.38 60.15) (end 87.89 66.64) (width 1) (layer "B.Cu") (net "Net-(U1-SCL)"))
 (segment (start 80.03 49.68) (end 80 49.71) (width 0.2) (layer "B.Cu") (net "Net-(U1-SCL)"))
 (segment (start 82.57 57.5) (end 82.57 60.07) (width 1) (layer "B.Cu") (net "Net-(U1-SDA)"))
 (segment (start 82.57 57.5) (end 82.57 49.68) (width 1) (layer "B.Cu") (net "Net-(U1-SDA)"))
 (segment (start 89.98 57.5) (end 94.38 53.1) (width 1) (layer "B.Cu") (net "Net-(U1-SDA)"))
 (segment (start 82.57 60.07) (end 85.35 62.85) (width 1) (layer "B.Cu") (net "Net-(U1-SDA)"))
 (segment (start 85.35 62.85) (end 85.35 66.64) (width 1) (layer "B.Cu") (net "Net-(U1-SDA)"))
 (segment (start 82.57 57.5) (end 89.98 57.5) (width 1) (layer "B.Cu") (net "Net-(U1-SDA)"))
 (segment (start 104 72.64) (end 101 72.64) (width 1) (layer "B.Cu") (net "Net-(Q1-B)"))
 (segment (start 105.27 70.34) (end 105.27 71.37) (width 1) (layer "B.Cu") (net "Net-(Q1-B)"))
 (segment (start 105.27 71.37) (end 104 72.64) (width 1) (layer "B.Cu") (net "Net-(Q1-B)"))
 (segment (start 100.54 72.18) (end 100.54 70.34) (width 1) (layer "B.Cu") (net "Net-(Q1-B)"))
 (segment (start 101 72.64) (end 100.54 72.18) (width 1) (layer "B.Cu") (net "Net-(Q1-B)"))
 (segment (start 93 76.39) (end 95.25 78.64) (width 1) (layer "B.Cu") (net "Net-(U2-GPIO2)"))
 (segment (start 95.25 78.64) (end 113 78.64) (width 1) (layer "B.Cu") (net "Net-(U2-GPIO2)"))
 (segment (start 113.84 65.8) (end 115 66.96) (width 1) (layer "B.Cu") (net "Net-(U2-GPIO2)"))
 (segment (start 113 78.64) (end 115 76.64) (width 1) (layer "B.Cu") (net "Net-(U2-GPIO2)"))
 (segment (start 115 66.96) (end 115 76.64) (width 1) (layer "B.Cu") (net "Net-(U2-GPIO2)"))
 (segment (start 113.84 65.8) (end 109.62 65.8) (width 1) (layer "B.Cu") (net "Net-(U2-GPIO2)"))
 (segment (start 109.62 72.38) (end 109.62 68.34) (width 1) (layer "B.Cu") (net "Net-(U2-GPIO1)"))
 (segment (start 105.61 76.39) (end 109.62 72.38) (width 1) (layer "B.Cu") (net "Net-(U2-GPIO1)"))
 (segment (start 102.75 76.39) (end 105.61 76.39) (width 1) (layer "B.Cu") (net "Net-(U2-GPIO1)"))
 (segment (start 67.46 78.64) (end 73.46 72.64) (width 1) (layer "B.Cu") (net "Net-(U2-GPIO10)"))
 (segment (start 87.54 72.64) (end 94.38 65.8) (width 1) (layer "B.Cu") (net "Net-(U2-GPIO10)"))
 (segment (start 73.46 72.64) (end 87.54 72.64) (width 1) (layer "B.Cu") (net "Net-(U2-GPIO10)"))
 (segment (start 80.46 77.5) (end 82.96 75) (width 1) (layer "B.Cu") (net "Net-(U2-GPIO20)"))
 (segment (start 80.46 77.5) (end 80.46 77.225787) (width 1) (layer "B.Cu") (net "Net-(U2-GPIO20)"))
 (segment (start 80.46 78.64) (end 80.46 77.5) (width 1) (layer "B.Cu") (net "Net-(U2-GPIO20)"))
 (segment (start 87.72 75) (end 94.38 68.34) (width 1) (layer "B.Cu") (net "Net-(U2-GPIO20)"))
 (segment (start 82.96 75) (end 87.72 75) (width 1) (layer "B.Cu") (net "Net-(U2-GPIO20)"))
 (segment (start 98 70.34) (end 94.92 70.34) (width 1) (layer "B.Cu") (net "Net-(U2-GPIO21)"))
 (segment (start 94.92 70.34) (end 94.38 70.88) (width 1) (layer "B.Cu") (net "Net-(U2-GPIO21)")))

